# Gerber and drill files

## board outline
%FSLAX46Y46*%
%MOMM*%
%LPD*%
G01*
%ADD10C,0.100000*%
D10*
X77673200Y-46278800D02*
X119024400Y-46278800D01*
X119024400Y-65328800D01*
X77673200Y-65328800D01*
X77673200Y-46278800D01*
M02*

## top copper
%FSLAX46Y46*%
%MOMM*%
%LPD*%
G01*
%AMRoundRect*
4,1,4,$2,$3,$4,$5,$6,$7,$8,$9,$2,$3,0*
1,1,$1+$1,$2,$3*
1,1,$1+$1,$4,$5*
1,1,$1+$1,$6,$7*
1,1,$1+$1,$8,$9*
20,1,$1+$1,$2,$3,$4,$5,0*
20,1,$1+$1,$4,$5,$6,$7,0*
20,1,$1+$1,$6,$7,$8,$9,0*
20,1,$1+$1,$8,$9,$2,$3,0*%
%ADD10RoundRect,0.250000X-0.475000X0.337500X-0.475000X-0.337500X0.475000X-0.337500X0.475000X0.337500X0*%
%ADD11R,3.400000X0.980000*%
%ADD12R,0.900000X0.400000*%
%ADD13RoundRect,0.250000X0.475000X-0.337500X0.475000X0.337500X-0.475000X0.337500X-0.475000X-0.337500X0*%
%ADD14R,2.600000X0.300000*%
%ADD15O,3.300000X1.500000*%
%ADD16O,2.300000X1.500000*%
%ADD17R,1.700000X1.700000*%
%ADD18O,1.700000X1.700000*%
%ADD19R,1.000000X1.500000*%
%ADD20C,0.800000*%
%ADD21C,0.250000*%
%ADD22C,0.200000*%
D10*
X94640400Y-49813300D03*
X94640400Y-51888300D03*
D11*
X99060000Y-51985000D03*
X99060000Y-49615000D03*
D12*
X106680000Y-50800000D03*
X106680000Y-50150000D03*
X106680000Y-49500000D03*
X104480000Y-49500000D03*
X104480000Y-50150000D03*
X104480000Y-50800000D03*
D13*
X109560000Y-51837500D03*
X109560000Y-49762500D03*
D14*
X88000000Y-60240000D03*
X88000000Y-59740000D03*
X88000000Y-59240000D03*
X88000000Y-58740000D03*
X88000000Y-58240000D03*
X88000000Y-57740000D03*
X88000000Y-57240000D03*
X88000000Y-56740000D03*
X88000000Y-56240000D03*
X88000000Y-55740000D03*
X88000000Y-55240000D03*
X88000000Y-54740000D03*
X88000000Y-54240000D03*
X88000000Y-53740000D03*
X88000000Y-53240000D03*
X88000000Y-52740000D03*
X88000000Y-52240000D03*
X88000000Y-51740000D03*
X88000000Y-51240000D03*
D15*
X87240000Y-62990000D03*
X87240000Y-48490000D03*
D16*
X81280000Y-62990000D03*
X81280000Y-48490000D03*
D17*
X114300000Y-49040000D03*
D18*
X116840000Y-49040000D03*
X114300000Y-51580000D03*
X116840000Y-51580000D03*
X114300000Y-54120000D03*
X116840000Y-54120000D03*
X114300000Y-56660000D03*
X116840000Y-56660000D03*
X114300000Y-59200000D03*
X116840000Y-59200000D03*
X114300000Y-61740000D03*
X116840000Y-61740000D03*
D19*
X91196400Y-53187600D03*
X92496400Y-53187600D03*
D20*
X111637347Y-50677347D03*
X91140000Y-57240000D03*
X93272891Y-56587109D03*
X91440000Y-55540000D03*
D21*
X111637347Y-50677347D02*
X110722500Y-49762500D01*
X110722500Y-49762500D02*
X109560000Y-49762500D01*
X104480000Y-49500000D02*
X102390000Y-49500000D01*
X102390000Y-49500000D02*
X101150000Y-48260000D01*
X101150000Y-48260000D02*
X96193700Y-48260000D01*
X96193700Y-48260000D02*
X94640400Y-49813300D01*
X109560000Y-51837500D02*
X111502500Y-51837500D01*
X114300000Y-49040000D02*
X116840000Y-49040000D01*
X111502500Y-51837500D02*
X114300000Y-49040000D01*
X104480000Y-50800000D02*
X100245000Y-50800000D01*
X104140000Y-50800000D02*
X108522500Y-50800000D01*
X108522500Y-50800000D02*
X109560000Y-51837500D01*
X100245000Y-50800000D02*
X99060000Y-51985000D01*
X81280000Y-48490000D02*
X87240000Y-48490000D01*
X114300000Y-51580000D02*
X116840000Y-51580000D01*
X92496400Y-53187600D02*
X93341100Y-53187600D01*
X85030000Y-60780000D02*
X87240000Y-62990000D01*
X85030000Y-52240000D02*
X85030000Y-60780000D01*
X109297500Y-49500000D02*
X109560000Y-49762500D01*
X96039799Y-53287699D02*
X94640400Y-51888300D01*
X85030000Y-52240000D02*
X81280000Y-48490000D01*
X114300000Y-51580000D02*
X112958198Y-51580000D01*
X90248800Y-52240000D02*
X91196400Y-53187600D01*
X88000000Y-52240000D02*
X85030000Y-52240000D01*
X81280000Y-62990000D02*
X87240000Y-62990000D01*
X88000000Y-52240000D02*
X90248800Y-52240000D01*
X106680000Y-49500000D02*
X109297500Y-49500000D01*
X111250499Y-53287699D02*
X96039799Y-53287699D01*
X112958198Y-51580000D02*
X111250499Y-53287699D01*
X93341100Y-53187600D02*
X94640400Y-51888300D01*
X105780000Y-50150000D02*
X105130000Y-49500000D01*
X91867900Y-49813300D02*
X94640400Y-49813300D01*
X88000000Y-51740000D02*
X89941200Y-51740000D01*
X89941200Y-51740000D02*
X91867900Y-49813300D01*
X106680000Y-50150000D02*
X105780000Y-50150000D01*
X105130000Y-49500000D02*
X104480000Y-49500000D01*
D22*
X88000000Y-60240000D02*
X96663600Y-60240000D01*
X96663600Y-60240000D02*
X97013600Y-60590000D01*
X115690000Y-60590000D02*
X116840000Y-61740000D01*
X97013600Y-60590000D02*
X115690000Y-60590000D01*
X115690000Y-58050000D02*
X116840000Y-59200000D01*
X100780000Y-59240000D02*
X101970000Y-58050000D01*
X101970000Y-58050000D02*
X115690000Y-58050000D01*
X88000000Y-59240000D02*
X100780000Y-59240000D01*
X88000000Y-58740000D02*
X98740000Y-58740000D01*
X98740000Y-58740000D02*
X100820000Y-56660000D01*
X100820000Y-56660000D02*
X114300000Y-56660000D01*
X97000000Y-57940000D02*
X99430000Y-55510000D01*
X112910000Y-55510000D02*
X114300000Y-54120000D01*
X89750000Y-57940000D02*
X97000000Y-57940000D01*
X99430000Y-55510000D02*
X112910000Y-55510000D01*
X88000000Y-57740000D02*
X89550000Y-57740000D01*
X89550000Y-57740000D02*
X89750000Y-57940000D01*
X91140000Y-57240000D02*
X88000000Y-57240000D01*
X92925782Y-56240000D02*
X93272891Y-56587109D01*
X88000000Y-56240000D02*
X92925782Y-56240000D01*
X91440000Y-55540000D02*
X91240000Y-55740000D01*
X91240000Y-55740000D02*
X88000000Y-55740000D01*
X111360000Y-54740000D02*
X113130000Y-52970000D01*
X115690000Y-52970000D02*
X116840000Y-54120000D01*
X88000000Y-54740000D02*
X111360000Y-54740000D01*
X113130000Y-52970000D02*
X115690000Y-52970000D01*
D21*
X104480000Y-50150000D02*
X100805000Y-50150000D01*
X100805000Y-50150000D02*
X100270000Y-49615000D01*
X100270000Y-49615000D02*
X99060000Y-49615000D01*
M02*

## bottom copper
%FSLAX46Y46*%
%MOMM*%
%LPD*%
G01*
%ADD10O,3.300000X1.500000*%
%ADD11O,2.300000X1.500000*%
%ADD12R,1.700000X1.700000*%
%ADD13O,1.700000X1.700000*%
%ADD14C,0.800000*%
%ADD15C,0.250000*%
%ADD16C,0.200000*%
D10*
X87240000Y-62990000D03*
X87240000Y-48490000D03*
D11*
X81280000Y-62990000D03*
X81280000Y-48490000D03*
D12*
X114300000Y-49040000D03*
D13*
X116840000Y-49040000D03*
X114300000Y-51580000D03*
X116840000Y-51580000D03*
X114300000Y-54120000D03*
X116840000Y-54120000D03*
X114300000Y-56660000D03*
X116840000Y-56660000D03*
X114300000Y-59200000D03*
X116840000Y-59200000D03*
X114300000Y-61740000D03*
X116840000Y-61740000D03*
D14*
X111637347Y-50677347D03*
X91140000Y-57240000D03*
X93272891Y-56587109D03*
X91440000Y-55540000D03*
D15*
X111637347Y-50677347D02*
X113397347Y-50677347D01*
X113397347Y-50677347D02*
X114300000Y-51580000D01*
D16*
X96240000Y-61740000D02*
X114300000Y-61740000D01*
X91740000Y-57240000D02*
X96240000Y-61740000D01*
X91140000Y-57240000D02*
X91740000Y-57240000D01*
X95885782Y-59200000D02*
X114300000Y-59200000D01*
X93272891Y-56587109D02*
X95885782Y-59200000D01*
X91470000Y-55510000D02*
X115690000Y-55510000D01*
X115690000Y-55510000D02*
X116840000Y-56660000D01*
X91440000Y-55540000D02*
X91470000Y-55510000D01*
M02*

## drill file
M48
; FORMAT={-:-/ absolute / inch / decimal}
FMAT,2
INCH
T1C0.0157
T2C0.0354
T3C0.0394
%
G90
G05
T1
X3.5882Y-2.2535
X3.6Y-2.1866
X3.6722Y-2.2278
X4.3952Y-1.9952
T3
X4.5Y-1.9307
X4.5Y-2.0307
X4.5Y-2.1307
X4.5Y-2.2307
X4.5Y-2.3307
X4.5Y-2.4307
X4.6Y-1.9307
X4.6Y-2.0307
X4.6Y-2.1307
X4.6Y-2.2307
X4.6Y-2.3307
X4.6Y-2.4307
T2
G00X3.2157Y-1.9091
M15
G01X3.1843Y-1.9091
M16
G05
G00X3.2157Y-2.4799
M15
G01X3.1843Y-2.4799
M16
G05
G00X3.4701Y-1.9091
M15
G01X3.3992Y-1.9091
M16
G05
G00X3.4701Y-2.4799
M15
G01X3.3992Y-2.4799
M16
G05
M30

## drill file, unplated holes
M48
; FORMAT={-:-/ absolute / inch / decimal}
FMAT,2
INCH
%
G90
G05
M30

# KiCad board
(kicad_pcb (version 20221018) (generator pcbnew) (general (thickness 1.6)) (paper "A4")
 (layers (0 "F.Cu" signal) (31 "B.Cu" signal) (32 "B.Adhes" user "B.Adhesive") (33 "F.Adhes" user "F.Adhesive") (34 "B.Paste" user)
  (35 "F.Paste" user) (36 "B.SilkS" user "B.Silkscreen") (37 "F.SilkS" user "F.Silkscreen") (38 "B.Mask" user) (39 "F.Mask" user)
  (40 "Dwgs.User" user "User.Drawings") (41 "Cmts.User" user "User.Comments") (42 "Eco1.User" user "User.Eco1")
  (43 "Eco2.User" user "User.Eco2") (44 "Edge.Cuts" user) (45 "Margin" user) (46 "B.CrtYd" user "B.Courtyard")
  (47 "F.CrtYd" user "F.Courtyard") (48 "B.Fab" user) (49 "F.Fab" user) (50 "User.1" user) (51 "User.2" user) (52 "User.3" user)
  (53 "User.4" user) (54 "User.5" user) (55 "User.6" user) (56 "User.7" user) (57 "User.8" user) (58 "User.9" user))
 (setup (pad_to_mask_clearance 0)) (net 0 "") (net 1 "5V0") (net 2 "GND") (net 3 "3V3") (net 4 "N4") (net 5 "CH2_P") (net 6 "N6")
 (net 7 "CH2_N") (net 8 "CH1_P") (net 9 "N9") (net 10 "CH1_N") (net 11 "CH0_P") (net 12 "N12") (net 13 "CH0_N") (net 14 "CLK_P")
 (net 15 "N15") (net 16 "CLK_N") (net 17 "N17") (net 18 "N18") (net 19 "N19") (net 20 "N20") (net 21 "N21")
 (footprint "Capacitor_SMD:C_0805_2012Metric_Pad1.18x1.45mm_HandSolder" (layer "F.Cu") (at 94.6404 50.8508 -90)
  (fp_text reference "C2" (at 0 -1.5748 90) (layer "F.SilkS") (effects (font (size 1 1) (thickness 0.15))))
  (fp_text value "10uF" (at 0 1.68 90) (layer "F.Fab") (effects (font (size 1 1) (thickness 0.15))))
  (pad "1" smd roundrect (at -1.0375 0 270) (size 1.175 1.45) (layers "F.Cu" "F.Paste" "F.Mask") (roundrect_rratio 0.2127659574)
   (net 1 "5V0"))
  (pad "2" smd roundrect (at 1.0375 0 270) (size 1.175 1.45) (layers "F.Cu" "F.Paste" "F.Mask") (roundrect_rratio 0.2127659574)
   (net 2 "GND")))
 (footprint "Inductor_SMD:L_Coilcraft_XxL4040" (layer "F.Cu") (at 99.06 50.8 90)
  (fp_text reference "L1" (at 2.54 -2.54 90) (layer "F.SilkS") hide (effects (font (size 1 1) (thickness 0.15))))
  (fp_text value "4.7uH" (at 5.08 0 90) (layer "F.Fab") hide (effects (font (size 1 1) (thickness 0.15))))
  (pad "1" smd rect (at -1.185 0 90) (size 0.98 3.4) (layers "F.Cu" "F.Paste" "F.Mask") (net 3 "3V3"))
  (pad "2" smd rect (at 1.185 0 90) (size 0.98 3.4) (layers "F.Cu" "F.Paste" "F.Mask") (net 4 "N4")))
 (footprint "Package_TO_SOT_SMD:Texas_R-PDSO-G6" (layer "F.Cu") (at 105.58 50.15 180)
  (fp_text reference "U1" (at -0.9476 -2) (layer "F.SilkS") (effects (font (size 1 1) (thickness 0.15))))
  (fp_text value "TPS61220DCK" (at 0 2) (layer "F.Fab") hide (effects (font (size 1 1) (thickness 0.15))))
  (pad "1" smd rect (at -1.1 -0.65 180) (size 0.9 0.4) (layers "F.Cu" "F.Paste" "F.Mask") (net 3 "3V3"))
  (pad "2" smd rect (at -1.1 0 180) (size 0.9 0.4) (layers "F.Cu" "F.Paste" "F.Mask") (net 1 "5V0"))
  (pad "3" smd rect (at -1.1 0.65 180) (size 0.9 0.4) (layers "F.Cu" "F.Paste" "F.Mask") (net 2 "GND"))
  (pad "4" smd rect (at 1.1 0.65 180) (size 0.9 0.4) (layers "F.Cu" "F.Paste" "F.Mask") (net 1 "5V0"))
  (pad "5" smd rect (at 1.1 0 180) (size 0.9 0.4) (layers "F.Cu" "F.Paste" "F.Mask") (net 4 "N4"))
  (pad "6" smd rect (at 1.1 -0.65 180) (size 0.9 0.4) (layers "F.Cu" "F.Paste" "F.Mask") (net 3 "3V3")))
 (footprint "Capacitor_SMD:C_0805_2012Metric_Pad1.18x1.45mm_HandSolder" (layer "F.Cu") (at 109.56 50.8 90)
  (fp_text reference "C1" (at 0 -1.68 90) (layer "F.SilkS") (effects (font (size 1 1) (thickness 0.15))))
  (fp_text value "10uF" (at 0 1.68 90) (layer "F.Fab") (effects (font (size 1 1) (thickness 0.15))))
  (pad "1" smd roundrect (at -1.0375 0 90) (size 1.175 1.45) (layers "F.Cu" "F.Paste" "F.Mask") (roundrect_rratio 0.2127659574)
   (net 3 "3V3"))
  (pad "2" smd roundrect (at 1.0375 0 90) (size 1.175 1.45) (layers "F.Cu" "F.Paste" "F.Mask") (roundrect_rratio 0.2127659574) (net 2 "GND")))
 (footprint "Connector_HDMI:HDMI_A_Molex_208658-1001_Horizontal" (layer "F.Cu") (at 84.715 55.74 180)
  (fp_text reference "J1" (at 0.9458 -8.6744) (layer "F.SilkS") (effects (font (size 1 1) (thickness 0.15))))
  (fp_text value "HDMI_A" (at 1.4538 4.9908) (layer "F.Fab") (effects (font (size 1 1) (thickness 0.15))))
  (pad "1" smd rect (at -3.285 -4.5 180) (size 2.6 0.3) (layers "F.Cu" "F.Paste" "F.Mask") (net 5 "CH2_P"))
  (pad "2" smd rect (at -3.285 -4 180) (size 2.6 0.3) (layers "F.Cu" "F.Paste" "F.Mask") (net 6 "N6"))
  (pad "3" smd rect (at -3.285 -3.5 180) (size 2.6 0.3) (layers "F.Cu" "F.Paste" "F.Mask") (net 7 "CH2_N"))
  (pad "4" smd rect (at -3.285 -3 180) (size 2.6 0.3) (layers "F.Cu" "F.Paste" "F.Mask") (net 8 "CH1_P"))
  (pad "5" smd rect (at -3.285 -2.5 180) (size 2.6 0.3) (layers "F.Cu" "F.Paste" "F.Mask") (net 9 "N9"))
  (pad "6" smd rect (at -3.285 -2 180) (size 2.6 0.3) (layers "F.Cu" "F.Paste" "F.Mask") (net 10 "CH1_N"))
  (pad "7" smd rect (at -3.285 -1.5 180) (size 2.6 0.3) (layers "F.Cu" "F.Paste" "F.Mask") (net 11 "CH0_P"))
  (pad "8" smd rect (at -3.285 -1 180) (size 2.6 0.3) (layers "F.Cu" "F.Paste" "F.Mask") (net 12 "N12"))
  (pad "9" smd rect (at -3.285 -0.5 180) (size 2.6 0.3) (layers "F.Cu" "F.Paste" "F.Mask") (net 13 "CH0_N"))
  (pad "10" smd rect (at -3.285 0 180) (size 2.6 0.3) (layers "F.Cu" "F.Paste" "F.Mask") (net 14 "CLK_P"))
  (pad "11" smd rect (at -3.285 0.5 180) (size 2.6 0.3) (layers "F.Cu" "F.Paste" "F.Mask") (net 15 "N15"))
  (pad "12" smd rect (at -3.285 1 180) (size 2.6 0.3) (layers "F.Cu" "F.Paste" "F.Mask") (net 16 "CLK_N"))
  (pad "13" smd rect (at -3.285 1.5 180) (size 2.6 0.3) (layers "F.Cu" "F.Paste" "F.Mask") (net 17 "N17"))
  (pad "14" smd rect (at -3.285 2 180) (size 2.6 0.3) (layers "F.Cu" "F.Paste" "F.Mask") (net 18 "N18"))
  (pad "15" smd rect (at -3.285 2.5 180) (size 2.6 0.3) (layers "F.Cu" "F.Paste" "F.Mask") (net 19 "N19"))
  (pad "16" smd rect (at -3.285 3 180) (size 2.6 0.3) (layers "F.Cu" "F.Paste" "F.Mask") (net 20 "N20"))
  (pad "17" smd rect (at -3.285 3.5 180) (size 2.6 0.3) (layers "F.Cu" "F.Paste" "F.Mask") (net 2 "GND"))
  (pad "18" smd rect (at -3.285 4 180) (size 2.6 0.3) (layers "F.Cu" "F.Paste" "F.Mask") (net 1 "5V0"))
  (pad "19" smd rect (at -3.285 4.5 180) (size 2.6 0.3) (layers "F.Cu" "F.Paste" "F.Mask") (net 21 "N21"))
  (pad "SH" thru_hole oval (at -2.525 -7.25 180) (size 3.3 1.5) (drill oval 2.7 0.9) (layers "*.Cu" "*.Mask") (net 2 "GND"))
  (pad "SH" thru_hole oval (at -2.525 7.25 180) (size 3.3 1.5) (drill oval 2.7 0.9) (layers "*.Cu" "*.Mask") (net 2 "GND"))
  (pad "SH" thru_hole oval (at 3.435 -7.25 180) (size 2.3 1.5) (drill oval 1.7 0.9) (layers "*.Cu" "*.Mask") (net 2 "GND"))
  (pad "SH" thru_hole oval (at 3.435 7.25 180) (size 2.3 1.5) (drill oval 1.7 0.9) (layers "*.Cu" "*.Mask") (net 2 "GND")))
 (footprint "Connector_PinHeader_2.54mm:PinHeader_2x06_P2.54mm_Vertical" (layer "F.Cu") (at 114.3 49.04)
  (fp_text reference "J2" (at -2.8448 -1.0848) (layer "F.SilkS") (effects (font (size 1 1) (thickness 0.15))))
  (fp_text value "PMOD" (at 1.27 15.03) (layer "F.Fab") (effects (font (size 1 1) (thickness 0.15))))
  (pad "1" thru_hole rect (at 0 0) (size 1.7 1.7) (drill 1) (layers "*.Cu" "*.Mask") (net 3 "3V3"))
  (pad "2" thru_hole oval (at 2.54 0) (size 1.7 1.7) (drill 1) (layers "*.Cu" "*.Mask") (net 3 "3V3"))
  (pad "3" thru_hole oval (at 0 2.54) (size 1.7 1.7) (drill 1) (layers "*.Cu" "*.Mask") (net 2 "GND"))
  (pad "4" thru_hole oval (at 2.54 2.54) (size 1.7 1.7) (drill 1) (layers "*.Cu" "*.Mask") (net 2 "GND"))
  (pad "5" thru_hole oval (at 0 5.08) (size 1.7 1.7) (drill 1) (layers "*.Cu" "*.Mask") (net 10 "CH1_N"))
  (pad "6" thru_hole oval (at 2.54 5.08) (size 1.7 1.7) (drill 1) (layers "*.Cu" "*.Mask") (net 16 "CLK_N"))
  (pad "7" thru_hole oval (at 0 7.62) (size 1.7 1.7) (drill 1) (layers "*.Cu" "*.Mask") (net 8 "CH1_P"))
  (pad "8" thru_hole oval (at 2.54 7.62) (size 1.7 1.7) (drill 1) (layers "*.Cu" "*.Mask") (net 14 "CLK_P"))
  (pad "9" thru_hole oval (at 0 10.16) (size 1.7 1.7) (drill 1) (layers "*.Cu" "*.Mask") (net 13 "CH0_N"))
  (pad "10" thru_hole oval (at 2.54 10.16) (size 1.7 1.7) (drill 1) (layers "*.Cu" "*.Mask") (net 7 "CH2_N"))
  (pad "11" thru_hole oval (at 0 12.7) (size 1.7 1.7) (drill 1) (layers "*.Cu" "*.Mask") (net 11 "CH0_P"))
  (pad "12" thru_hole oval (at 2.54 12.7) (size 1.7 1.7) (drill 1) (layers "*.Cu" "*.Mask") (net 5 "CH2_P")))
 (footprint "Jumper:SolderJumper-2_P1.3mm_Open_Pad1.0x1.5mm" (layer "F.Cu") (at 91.8464 53.1876)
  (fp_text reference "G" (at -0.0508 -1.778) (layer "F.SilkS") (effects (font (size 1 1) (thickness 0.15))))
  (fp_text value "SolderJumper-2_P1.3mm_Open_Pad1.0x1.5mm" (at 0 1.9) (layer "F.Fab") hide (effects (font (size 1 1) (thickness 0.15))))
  (pad "1" smd rect (at -0.65 0) (size 1 1.5) (layers "F.Cu" "F.Mask") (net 2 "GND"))
  (pad "2" smd rect (at 0.65 0) (size 1 1.5) (layers "F.Cu" "F.Mask") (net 2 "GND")))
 (gr_rect (start 77.6732 46.2788) (end 119.0244 65.3288) (stroke (width 0.1) (type default)) (fill none) (layer "Edge.Cuts"))
 (segment (start 109.56 51.8375) (end 111.5025 51.8375) (width 0.25) (layer "F.Cu") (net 3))
 (segment (start 114.3 49.04) (end 116.84 49.04) (width 0.25) (layer "F.Cu") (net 3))
 (segment (start 111.5025 51.8375) (end 114.3 49.04) (width 0.25) (layer "F.Cu") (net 3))
 (segment (start 104.48 50.8) (end 100.245 50.8) (width 0.25) (layer "F.Cu") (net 3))
 (segment (start 104.14 50.8) (end 108.5225 50.8) (width 0.25) (layer "F.Cu") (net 3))
 (segment (start 108.5225 50.8) (end 109.56 51.8375) (width 0.25) (layer "F.Cu") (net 3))
 (segment (start 100.245 50.8) (end 99.06 51.985) (width 0.25) (layer "F.Cu") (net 3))
 (segment (start 81.28 48.49) (end 87.24 48.49) (width 0.25) (layer "F.Cu") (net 2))
 (segment (start 114.3 51.58) (end 116.84 51.58) (width 0.25) (layer "F.Cu") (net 2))
 (segment (start 92.4964 53.1876) (end 93.3411 53.1876) (width 0.25) (layer "F.Cu") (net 2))
 (segment (start 85.03 60.78) (end 87.24 62.99) (width 0.25) (layer "F.Cu") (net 2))
 (segment (start 85.03 52.24) (end 85.03 60.78) (width 0.25) (layer "F.Cu") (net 2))
 (segment (start 109.2975 49.5) (end 109.56 49.7625) (width 0.25) (layer "F.Cu") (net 2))
 (segment (start 96.039799 53.287699) (end 94.6404 51.8883) (width 0.25) (layer "F.Cu") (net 2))
 (segment (start 111.637347 50.677347) (end 110.7225 49.7625) (width 0.25) (layer "F.Cu") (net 2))
 (segment (start 110.7225 49.7625) (end 109.56 49.7625) (width 0.25) (layer "F.Cu") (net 2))
 (segment (start 85.03 52.24) (end 81.28 48.49) (width 0.25) (layer "F.Cu") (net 2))
 (segment (start 114.3 51.58) (end 112.958198 51.58) (width 0.25) (layer "F.Cu") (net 2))
 (segment (start 90.2488 52.24) (end 91.1964 53.1876) (width 0.25) (layer "F.Cu") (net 2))
 (segment (start 88 52.24) (end 85.03 52.24) (width 0.25) (layer "F.Cu") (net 2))
 (segment (start 81.28 62.99) (end 87.24 62.99) (width 0.25) (layer "F.Cu") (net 2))
 (segment (start 88 52.24) (end 90.2488 52.24) (width 0.25) (layer "F.Cu") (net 2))
 (segment (start 106.68 49.5) (end 109.2975 49.5) (width 0.25) (layer "F.Cu") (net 2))
 (segment (start 111.250499 53.287699) (end 96.039799 53.287699) (width 0.25) (layer "F.Cu") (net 2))
 (segment (start 112.958198 51.58) (end 111.250499 53.287699) (width 0.25) (layer "F.Cu") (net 2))
 (segment (start 93.3411 53.1876) (end 94.6404 51.8883) (width 0.25) (layer "F.Cu") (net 2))
 (via (at 111.637347 50.677347) (size 0.8) (drill 0.4) (layers "F.Cu" "B.Cu") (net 2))
 (segment (start 113.397347 50.677347) (end 114.3 51.58) (width 0.25) (layer "B.Cu") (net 2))
 (segment (start 111.637347 50.677347) (end 113.397347 50.677347) (width 0.25) (layer "B.Cu") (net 2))
 (segment (start 105.78 50.15) (end 105.13 49.5) (width 0.25) (layer "F.Cu") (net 1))
 (segment (start 104.48 49.5) (end 102.39 49.5) (width 0.25) (layer "F.Cu") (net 1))
 (segment (start 91.8679 49.8133) (end 94.6404 49.8133) (width 0.25) (layer "F.Cu") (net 1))
 (segment (start 88 51.74) (end 89.9412 51.74) (width 0.25) (layer "F.Cu") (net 1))
 (segment (start 89.9412 51.74) (end 91.8679 49.8133) (width 0.25) (layer "F.Cu") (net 1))
 (segment (start 102.39 49.5) (end 101.15 48.26) (width 0.25) (layer "F.Cu") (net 1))
 (segment (start 106.68 50.15) (end 105.78 50.15) (width 0.25) (layer "F.Cu") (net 1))
 (segment (start 96.1937 48.26) (end 94.6404 49.8133) (width 0.25) (layer "F.Cu") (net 1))
 (segment (start 101.15 48.26) (end 96.1937 48.26) (width 0.25) (layer "F.Cu") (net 1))
 (segment (start 105.13 49.5) (end 104.48 49.5) (width 0.25) (layer "F.Cu") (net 1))
 (segment (start 88 60.24) (end 96.6636 60.24) (width 0.2) (layer "F.Cu") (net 5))
 (segment (start 96.6636 60.24) (end 97.0136 60.59) (width 0.2) (layer "F.Cu") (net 5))
 (segment (start 115.69 60.59) (end 116.84 61.74) (width 0.2) (layer "F.Cu") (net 5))
 (segment (start 97.0136 60.59) (end 115.69 60.59) (width 0.2) (layer "F.Cu") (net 5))
 (segment (start 115.69 58.05) (end 116.84 59.2) (width 0.2) (layer "F.Cu") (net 7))
 (segment (start 100.78 59.24) (end 101.97 58.05) (width 0.2) (layer "F.Cu") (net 7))
 (segment (start 101.97 58.05) (end 115.69 58.05) (width 0.2) (layer "F.Cu") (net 7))
 (segment (start 88 59.24) (end 100.78 59.24) (width 0.2) (layer "F.Cu") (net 7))
 (segment (start 88 58.74) (end 98.74 58.74) (width 0.2) (layer "F.Cu") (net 8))
 (segment (start 98.74 58.74) (end 100.82 56.66) (width 0.2) (layer "F.Cu") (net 8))
 (segment (start 100.82 56.66) (end 114.3 56.66) (width 0.2) (layer "F.Cu") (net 8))
 (segment (start 97 57.94) (end 99.43 55.51) (width 0.2) (layer "F.Cu") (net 10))
 (segment (start 112.91 55.51) (end 114.3 54.12) (width 0.2) (layer "F.Cu") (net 10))
 (segment (start 89.75 57.94) (end 97 57.94) (width 0.2) (layer "F.Cu") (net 10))
 (segment (start 99.43 55.51) (end 112.91 55.51) (width 0.2) (layer "F.Cu") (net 10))
 (segment (start 88 57.74) (end 89.55 57.74) (width 0.2) (layer "F.Cu") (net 10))
 (segment (start 89.55 57.74) (end 89.75 57.94) (width 0.2) (layer "F.Cu") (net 10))
 (segment (start 91.14 57.24) (end 88 57.24) (width 0.2) (layer "F.Cu") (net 11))
 (via (at 91.14 57.24) (size 0.8) (drill 0.4) (layers "F.Cu" "B.Cu") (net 11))
 (segment (start 96.24 61.74) (end 114.3 61.74) (width 0.2) (layer "B.Cu") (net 11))
 (segment (start 91.74 57.24) (end 96.24 61.74) (width 0.2) (layer "B.Cu") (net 11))
 (segment (start 91.14 57.24) (end 91.74 57.24) (width 0.2) (layer "B.Cu") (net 11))
 (segment (start 92.925782 56.24) (end 93.272891 56.587109) (width 0.2) (layer "F.Cu") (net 13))
 (segment (start 88 56.24) (end 92.925782 56.24) (width 0.2) (layer "F.Cu") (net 13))
 (via (at 93.272891 56.587109) (size 0.8) (drill 0.4) (layers "F.Cu" "B.Cu") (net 13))
 (segment (start 95.885782 59.2) (end 114.3 59.2) (width 0.2) (layer "B.Cu") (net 13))
 (segment (start 93.272891 56.587109) (end 95.885782 59.2) (width 0.2) (layer "B.Cu") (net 13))
 (segment (start 91.44 55.54) (end 91.24 55.74) (width 0.2) (layer "F.Cu") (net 14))
 (segment (start 91.24 55.74) (end 88 55.74) (width 0.2) (layer "F.Cu") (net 14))
 (via (at 91.44 55.54) (size 0.8) (drill 0.4) (layers "F.Cu" "B.Cu") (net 14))
 (segment (start 91.47 55.51) (end 115.69 55.51) (width 0.2) (layer "B.Cu") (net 14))
 (segment (start 115.69 55.51) (end 116.84 56.66) (width 0.2) (layer "B.Cu") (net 14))
 (segment (start 91.44 55.54) (end 91.47 55.51) (width 0.2) (layer "B.Cu") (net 14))
 (segment (start 111.36 54.74) (end 113.13 52.97) (width 0.2) (layer "F.Cu") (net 16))
 (segment (start 115.69 52.97) (end 116.84 54.12) (width 0.2) (layer "F.Cu") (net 16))
 (segment (start 88 54.74) (end 111.36 54.74) (width 0.2) (layer "F.Cu") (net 16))
 (segment (start 113.13 52.97) (end 115.69 52.97) (width 0.2) (layer "F.Cu") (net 16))
 (segment (start 104.48 50.15) (end 100.805 50.15) (width 0.25) (layer "F.Cu") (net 4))
 (segment (start 100.805 50.15) (end 100.27 49.615) (width 0.25) (layer "F.Cu") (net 4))
 (segment (start 100.27 49.615) (end 99.06 49.615) (width 0.25) (layer "F.Cu") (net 4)))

